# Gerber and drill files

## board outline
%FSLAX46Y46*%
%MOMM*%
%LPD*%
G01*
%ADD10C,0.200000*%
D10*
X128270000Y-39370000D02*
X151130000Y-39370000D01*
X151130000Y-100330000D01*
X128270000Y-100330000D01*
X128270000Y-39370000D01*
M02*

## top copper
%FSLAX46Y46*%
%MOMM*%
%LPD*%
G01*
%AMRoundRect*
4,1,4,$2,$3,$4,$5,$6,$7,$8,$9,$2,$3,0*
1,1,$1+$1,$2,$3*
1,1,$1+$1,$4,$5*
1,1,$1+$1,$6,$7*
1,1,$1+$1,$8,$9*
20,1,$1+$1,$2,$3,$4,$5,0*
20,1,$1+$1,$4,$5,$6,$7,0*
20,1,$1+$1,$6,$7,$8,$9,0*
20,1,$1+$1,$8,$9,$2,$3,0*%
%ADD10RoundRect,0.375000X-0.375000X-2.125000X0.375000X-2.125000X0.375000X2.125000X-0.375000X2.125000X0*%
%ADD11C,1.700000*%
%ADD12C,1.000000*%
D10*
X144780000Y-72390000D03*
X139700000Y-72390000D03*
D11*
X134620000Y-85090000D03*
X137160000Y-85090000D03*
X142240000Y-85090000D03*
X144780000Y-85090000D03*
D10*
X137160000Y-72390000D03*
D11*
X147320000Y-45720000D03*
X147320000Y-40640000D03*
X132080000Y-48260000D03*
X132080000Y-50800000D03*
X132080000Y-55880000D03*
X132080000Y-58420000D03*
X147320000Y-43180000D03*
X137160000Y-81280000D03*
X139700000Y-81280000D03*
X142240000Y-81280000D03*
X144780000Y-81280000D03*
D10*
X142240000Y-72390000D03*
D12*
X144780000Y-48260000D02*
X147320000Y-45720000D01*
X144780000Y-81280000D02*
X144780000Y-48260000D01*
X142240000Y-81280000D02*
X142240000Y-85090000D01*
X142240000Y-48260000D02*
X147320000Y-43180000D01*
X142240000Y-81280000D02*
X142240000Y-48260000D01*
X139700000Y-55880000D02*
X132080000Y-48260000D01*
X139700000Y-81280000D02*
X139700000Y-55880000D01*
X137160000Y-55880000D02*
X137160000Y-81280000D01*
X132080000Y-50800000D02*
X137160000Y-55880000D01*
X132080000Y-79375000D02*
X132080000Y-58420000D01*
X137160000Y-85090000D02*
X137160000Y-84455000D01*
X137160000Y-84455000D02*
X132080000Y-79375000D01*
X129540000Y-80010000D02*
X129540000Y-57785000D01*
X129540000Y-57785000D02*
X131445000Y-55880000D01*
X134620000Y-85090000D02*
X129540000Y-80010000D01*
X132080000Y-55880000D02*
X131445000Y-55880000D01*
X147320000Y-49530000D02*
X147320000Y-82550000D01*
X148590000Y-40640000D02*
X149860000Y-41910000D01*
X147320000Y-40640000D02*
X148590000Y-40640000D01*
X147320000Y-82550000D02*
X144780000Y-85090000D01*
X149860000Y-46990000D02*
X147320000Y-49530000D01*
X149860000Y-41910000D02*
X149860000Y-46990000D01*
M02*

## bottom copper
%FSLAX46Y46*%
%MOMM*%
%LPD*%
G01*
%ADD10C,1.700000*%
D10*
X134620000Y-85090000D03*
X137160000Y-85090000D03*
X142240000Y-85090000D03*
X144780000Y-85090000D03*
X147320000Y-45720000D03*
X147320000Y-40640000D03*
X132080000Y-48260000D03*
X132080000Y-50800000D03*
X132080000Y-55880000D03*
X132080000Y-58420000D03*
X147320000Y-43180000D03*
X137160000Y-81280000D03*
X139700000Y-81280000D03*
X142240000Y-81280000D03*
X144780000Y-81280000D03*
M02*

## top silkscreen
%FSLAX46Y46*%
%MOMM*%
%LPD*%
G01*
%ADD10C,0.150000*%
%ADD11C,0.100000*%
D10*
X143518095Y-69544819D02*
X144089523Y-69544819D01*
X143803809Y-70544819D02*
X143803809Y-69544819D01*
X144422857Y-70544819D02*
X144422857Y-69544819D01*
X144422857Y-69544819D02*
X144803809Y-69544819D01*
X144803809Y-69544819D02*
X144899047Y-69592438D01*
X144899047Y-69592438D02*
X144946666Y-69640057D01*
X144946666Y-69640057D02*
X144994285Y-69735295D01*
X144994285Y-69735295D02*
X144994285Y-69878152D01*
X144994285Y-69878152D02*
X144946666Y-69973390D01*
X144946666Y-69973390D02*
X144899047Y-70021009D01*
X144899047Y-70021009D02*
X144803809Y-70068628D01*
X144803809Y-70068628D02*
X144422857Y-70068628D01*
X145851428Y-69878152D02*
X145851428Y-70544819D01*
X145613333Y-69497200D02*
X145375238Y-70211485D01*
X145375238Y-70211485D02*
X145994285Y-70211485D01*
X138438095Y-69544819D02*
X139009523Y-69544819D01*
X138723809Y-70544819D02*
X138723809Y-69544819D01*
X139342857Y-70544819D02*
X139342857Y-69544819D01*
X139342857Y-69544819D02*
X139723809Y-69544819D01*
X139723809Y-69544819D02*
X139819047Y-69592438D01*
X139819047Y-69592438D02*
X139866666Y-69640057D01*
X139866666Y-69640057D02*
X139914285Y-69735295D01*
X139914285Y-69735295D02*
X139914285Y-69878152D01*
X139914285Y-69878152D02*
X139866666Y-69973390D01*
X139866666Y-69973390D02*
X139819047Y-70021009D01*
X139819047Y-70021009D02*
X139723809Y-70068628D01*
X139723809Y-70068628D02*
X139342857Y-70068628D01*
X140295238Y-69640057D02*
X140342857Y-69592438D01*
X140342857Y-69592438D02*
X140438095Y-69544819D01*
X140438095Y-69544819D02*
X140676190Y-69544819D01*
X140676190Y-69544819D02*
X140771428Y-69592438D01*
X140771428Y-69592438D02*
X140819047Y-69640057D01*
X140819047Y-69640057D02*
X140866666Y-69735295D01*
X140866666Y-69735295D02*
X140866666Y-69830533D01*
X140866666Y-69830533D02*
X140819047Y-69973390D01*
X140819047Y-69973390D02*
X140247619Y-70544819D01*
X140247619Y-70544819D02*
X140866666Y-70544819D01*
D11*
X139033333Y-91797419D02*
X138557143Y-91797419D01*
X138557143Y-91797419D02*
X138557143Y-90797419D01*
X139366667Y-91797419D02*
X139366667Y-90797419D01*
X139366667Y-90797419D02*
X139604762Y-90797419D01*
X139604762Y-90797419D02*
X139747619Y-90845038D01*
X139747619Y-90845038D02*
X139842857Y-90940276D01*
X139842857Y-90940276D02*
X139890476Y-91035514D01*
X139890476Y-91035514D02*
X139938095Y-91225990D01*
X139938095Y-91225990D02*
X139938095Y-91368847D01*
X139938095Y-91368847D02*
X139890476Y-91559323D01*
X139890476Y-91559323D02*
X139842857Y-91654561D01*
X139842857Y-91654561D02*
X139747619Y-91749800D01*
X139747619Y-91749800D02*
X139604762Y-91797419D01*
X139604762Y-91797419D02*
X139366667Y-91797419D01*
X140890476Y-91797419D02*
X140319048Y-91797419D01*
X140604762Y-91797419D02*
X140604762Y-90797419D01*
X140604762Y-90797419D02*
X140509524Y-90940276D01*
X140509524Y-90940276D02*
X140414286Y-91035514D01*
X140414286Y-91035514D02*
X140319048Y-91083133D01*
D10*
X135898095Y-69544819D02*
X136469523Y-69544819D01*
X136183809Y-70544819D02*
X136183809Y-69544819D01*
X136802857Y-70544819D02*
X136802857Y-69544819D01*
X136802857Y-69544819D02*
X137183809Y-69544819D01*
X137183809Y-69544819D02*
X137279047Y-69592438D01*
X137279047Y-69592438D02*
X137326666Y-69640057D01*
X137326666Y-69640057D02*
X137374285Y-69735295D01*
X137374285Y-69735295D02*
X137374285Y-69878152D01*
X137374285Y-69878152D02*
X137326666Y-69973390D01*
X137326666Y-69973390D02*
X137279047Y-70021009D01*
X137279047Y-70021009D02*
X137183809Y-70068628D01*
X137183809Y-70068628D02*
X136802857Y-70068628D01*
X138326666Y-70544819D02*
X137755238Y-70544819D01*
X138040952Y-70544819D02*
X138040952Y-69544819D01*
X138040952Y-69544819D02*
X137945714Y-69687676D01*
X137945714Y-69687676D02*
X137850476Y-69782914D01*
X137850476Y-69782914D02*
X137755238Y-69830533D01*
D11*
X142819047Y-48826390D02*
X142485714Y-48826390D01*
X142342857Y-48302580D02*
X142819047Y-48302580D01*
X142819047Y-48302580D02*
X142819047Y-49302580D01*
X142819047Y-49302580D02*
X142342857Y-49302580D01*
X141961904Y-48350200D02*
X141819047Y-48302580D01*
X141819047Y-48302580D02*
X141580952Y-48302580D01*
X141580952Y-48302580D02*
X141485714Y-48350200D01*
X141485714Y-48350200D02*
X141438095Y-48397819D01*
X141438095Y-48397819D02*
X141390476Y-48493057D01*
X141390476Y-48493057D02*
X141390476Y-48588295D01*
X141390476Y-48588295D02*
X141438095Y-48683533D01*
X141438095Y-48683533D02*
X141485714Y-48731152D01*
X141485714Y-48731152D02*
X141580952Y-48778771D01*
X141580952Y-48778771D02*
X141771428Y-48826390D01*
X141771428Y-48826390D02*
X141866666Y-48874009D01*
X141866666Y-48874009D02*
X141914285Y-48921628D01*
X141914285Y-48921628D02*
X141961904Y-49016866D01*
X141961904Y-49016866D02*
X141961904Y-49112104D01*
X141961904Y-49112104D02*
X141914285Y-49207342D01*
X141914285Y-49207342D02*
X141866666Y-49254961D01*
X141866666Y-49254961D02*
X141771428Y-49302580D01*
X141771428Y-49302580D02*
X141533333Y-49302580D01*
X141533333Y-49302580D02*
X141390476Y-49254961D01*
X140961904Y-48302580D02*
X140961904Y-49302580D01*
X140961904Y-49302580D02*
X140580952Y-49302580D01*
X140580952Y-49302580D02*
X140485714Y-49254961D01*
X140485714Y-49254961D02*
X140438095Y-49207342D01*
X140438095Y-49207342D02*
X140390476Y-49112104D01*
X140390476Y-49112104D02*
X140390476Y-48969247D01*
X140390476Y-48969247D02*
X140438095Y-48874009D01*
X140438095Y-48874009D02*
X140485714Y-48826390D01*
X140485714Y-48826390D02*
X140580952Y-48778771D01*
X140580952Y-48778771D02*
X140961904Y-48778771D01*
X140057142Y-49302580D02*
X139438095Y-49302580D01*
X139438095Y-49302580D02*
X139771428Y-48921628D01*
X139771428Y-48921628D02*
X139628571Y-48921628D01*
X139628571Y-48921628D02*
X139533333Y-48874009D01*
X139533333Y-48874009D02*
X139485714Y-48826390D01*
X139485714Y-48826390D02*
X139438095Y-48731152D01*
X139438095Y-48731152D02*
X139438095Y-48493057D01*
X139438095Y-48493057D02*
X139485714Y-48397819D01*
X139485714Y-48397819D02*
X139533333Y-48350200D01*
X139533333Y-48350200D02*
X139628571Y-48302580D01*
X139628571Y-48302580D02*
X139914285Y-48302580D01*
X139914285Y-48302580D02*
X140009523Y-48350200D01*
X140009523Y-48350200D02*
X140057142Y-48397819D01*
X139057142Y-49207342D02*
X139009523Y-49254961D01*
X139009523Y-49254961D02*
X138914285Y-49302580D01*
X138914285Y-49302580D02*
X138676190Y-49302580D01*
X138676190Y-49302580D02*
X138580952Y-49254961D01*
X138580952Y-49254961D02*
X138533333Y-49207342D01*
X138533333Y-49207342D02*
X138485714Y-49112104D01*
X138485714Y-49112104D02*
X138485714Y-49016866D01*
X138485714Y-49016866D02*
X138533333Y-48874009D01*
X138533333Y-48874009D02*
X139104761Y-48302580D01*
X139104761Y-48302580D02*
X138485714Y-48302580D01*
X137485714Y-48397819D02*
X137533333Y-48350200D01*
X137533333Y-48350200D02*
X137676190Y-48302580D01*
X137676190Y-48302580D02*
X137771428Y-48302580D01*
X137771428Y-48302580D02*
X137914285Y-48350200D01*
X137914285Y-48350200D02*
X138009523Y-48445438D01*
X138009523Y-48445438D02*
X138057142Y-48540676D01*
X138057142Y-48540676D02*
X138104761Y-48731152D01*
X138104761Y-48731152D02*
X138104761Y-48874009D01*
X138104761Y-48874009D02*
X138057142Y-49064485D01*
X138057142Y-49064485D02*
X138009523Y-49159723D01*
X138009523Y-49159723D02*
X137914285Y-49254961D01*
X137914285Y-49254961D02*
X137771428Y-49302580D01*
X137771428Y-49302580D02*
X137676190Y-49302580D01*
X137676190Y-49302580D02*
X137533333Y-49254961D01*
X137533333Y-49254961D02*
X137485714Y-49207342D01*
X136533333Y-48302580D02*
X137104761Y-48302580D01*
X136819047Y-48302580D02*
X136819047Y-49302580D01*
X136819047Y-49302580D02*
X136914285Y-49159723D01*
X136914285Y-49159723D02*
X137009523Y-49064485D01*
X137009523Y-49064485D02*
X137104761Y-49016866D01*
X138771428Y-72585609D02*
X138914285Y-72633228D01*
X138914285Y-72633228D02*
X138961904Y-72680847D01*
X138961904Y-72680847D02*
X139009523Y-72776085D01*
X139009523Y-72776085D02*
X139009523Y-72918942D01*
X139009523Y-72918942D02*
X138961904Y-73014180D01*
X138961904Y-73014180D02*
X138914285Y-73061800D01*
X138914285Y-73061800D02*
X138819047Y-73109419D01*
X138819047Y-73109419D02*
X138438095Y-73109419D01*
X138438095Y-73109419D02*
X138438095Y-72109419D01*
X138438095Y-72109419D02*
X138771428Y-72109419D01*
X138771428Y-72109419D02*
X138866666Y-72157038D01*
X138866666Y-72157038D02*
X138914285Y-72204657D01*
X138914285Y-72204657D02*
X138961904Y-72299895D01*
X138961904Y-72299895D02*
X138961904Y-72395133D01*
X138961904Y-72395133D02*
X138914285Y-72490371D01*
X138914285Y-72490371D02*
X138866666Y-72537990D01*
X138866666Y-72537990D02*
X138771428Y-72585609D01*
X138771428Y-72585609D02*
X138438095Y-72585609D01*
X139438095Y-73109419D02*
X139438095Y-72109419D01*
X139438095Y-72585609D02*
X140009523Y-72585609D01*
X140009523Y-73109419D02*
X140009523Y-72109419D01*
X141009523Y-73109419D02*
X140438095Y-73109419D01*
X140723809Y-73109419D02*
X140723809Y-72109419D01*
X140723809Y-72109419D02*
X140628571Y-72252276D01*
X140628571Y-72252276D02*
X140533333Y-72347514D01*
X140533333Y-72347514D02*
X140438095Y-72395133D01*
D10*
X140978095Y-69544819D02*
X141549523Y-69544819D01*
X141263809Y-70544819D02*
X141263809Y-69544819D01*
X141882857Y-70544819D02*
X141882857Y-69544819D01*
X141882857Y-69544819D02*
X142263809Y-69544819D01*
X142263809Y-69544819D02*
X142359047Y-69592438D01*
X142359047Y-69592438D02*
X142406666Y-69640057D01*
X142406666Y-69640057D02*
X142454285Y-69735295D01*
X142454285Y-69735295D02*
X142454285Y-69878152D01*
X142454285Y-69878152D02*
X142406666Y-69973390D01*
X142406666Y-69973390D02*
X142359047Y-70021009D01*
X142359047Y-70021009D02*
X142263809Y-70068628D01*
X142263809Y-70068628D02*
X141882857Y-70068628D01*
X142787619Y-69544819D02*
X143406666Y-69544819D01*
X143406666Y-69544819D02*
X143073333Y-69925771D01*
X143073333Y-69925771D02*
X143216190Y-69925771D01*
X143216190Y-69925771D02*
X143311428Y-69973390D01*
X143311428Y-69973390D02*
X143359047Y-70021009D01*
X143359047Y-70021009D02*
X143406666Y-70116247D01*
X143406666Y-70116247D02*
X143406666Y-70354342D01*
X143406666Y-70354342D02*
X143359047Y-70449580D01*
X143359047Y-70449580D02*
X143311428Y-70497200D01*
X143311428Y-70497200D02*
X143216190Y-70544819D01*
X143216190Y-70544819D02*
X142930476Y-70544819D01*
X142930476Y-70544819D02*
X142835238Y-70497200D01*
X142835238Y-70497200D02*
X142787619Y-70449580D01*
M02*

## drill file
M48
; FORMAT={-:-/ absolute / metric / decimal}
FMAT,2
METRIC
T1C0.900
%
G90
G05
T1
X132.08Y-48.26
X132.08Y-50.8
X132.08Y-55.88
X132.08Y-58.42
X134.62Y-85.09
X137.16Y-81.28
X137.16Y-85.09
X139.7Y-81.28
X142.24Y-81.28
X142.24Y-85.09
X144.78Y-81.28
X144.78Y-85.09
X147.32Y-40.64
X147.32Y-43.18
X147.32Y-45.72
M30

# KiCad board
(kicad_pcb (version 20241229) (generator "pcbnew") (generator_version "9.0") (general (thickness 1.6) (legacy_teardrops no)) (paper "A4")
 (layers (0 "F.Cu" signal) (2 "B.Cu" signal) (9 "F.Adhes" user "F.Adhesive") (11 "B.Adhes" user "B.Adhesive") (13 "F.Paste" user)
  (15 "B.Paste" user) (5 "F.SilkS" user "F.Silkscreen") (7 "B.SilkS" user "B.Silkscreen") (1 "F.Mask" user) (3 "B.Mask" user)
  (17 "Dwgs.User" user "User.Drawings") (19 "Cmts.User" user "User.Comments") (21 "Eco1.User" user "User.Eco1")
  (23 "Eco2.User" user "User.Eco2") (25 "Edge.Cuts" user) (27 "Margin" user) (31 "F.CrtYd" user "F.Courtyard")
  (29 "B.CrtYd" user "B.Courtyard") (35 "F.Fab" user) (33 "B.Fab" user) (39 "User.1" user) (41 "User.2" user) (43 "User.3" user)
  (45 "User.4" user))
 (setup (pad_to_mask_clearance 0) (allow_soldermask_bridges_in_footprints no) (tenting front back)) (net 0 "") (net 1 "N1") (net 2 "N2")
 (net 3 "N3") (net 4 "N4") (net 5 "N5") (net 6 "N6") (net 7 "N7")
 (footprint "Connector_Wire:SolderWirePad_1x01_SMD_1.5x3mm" (layer "F.Cu") (at 144.78 72.39)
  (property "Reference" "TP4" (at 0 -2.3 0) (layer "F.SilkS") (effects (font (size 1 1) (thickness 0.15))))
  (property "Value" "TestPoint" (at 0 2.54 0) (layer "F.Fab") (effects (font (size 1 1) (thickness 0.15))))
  (pad "1" smd roundrect (at 0 0) (size 1.5 5) (layers "F.Cu" "F.Mask") (roundrect_rratio 0.25) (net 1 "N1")))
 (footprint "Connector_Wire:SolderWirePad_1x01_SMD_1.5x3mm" (layer "F.Cu") (at 139.7 72.39)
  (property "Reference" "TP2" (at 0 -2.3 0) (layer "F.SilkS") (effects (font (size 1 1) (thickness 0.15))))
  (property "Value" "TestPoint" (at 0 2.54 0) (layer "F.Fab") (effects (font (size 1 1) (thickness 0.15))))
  (pad "1" smd roundrect (at 0 0) (size 1.5 5) (layers "F.Cu" "F.Mask") (roundrect_rratio 0.25) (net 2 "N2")))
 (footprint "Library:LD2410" (layer "F.Cu") (at 139.7 91.84)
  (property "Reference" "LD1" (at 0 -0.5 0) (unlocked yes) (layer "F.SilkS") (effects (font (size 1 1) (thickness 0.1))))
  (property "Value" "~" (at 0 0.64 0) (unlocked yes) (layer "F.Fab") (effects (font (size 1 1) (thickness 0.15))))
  (pad "1" thru_hole circle (at -5.08 -6.75 90) (size 1.7 1.7) (drill 0.9) (layers "*.Cu" "*.Mask") (remove_unused_layers yes)
   (keep_end_layers yes) (zone_layer_connections) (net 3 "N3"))
  (pad "2" thru_hole circle (at -2.54 -6.75 90) (size 1.7 1.7) (drill 0.9) (layers "*.Cu" "*.Mask") (remove_unused_layers yes)
   (keep_end_layers yes) (zone_layer_connections) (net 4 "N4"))
  (pad "4" thru_hole circle (at 2.54 -6.75 90) (size 1.7 1.7) (drill 0.9) (layers "*.Cu" "*.Mask") (remove_unused_layers yes)
   (keep_end_layers yes) (zone_layer_connections) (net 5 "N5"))
  (pad "5" thru_hole circle (at 5.08 -6.75 90) (size 1.7 1.7) (drill 0.9) (layers "*.Cu" "*.Mask") (remove_unused_layers yes)
   (keep_end_layers yes) (zone_layer_connections) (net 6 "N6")))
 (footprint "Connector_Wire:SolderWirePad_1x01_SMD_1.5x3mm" (layer "F.Cu") (at 137.16 72.39)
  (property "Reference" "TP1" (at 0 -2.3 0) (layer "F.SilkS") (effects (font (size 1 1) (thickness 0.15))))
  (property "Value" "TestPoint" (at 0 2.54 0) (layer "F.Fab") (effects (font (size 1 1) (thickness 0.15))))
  (pad "1" smd roundrect (at 0 0) (size 1.5 5) (layers "F.Cu" "F.Mask") (roundrect_rratio 0.25) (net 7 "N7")))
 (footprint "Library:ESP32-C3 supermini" (layer "F.Cu") (at 139.7 50.8 180)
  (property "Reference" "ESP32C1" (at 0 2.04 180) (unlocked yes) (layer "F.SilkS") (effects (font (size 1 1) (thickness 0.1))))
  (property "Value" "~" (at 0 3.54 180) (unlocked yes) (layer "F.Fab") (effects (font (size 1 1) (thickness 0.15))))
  (pad "3.3V" thru_hole circle (at -7.62 5.08 180) (size 1.7 1.7) (drill 0.9) (layers "*.Cu" "*.Mask") (remove_unused_layers yes)
   (keep_end_layers yes) (zone_layer_connections) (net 1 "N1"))
  (pad "5V" thru_hole circle (at -7.62 10.16 180) (size 1.7 1.7) (drill 0.9) (layers "*.Cu" "*.Mask") (remove_unused_layers yes)
   (keep_end_layers yes) (zone_layer_connections) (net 6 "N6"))
  (pad "8" thru_hole circle (at 7.62 2.54 180) (size 1.7 1.7) (drill 0.9) (layers "*.Cu" "*.Mask") (remove_unused_layers yes)
   (keep_end_layers yes) (zone_layer_connections) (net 2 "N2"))
  (pad "9" thru_hole circle (at 7.62 0 180) (size 1.7 1.7) (drill 0.9) (layers "*.Cu" "*.Mask") (remove_unused_layers yes)
   (keep_end_layers yes) (zone_layer_connections) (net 7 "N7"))
  (pad "20" thru_hole circle (at 7.62 -5.08 180) (size 1.7 1.7) (drill 0.9) (layers "*.Cu" "*.Mask") (remove_unused_layers yes)
   (keep_end_layers yes) (zone_layer_connections) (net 3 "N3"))
  (pad "21" thru_hole circle (at 7.62 -7.62 180) (size 1.7 1.7) (drill 0.9) (layers "*.Cu" "*.Mask") (remove_unused_layers yes)
   (keep_end_layers yes) (zone_layer_connections) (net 4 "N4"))
  (pad "GND" thru_hole circle (at -7.62 7.62 180) (size 1.7 1.7) (drill 0.9) (layers "*.Cu" "*.Mask") (remove_unused_layers yes)
   (keep_end_layers yes) (zone_layer_connections) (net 5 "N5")))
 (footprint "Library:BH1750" (layer "F.Cu") (at 139.7 73.152)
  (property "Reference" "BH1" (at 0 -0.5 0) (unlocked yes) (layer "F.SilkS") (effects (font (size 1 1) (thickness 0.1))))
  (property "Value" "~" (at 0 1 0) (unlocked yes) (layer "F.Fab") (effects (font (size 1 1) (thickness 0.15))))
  (pad "1" thru_hole circle (at -2.54 8.128 90) (size 1.7 1.7) (drill 0.9) (layers "*.Cu" "*.Mask") (remove_unused_layers yes)
   (keep_end_layers yes) (zone_layer_connections) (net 7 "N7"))
  (pad "2" thru_hole circle (at 0 8.128 90) (size 1.7 1.7) (drill 0.9) (layers "*.Cu" "*.Mask") (remove_unused_layers yes)
   (keep_end_layers yes) (zone_layer_connections) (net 2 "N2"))
  (pad "3" thru_hole circle (at 2.54 8.128 90) (size 1.7 1.7) (drill 0.9) (layers "*.Cu" "*.Mask") (remove_unused_layers yes)
   (keep_end_layers yes) (zone_layer_connections) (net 5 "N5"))
  (pad "4" thru_hole circle (at 5.08 8.128 90) (size 1.7 1.7) (drill 0.9) (layers "*.Cu" "*.Mask") (remove_unused_layers yes)
   (keep_end_layers yes) (zone_layer_connections) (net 1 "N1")))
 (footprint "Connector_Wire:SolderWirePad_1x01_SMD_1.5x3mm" (layer "F.Cu") (at 142.24 72.39)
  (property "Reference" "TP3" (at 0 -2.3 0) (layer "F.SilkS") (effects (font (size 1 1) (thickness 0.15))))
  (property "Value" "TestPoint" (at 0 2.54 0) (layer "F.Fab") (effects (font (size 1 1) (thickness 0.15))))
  (pad "1" smd roundrect (at 0 0) (size 1.5 5) (layers "F.Cu" "F.Mask") (roundrect_rratio 0.25) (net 5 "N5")))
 (gr_rect (start 128.27 39.37) (end 151.13 100.33) (stroke (width 0.2) (type solid)) (fill no) (layer "Edge.Cuts"))
 (segment (start 144.78 48.26) (end 147.32 45.72) (width 1) (layer "F.Cu") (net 1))
 (segment (start 144.78 81.28) (end 144.78 48.26) (width 1) (layer "F.Cu") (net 1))
 (segment (start 142.24 81.28) (end 142.24 85.09) (width 1) (layer "F.Cu") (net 5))
 (segment (start 142.24 48.26) (end 147.32 43.18) (width 1) (layer "F.Cu") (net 5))
 (segment (start 142.24 81.28) (end 142.24 48.26) (width 1) (layer "F.Cu") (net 5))
 (segment (start 139.7 55.88) (end 132.08 48.26) (width 1) (layer "F.Cu") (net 2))
 (segment (start 139.7 81.28) (end 139.7 55.88) (width 1) (layer "F.Cu") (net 2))
 (segment (start 137.16 55.88) (end 137.16 81.28) (width 1) (layer "F.Cu") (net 7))
 (segment (start 132.08 50.8) (end 137.16 55.88) (width 1) (layer "F.Cu") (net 7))
 (segment (start 132.08 79.375) (end 132.08 58.42) (width 1) (layer "F.Cu") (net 4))
 (segment (start 137.16 85.09) (end 137.16 84.455) (width 1) (layer "F.Cu") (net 4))
 (segment (start 137.16 84.455) (end 132.08 79.375) (width 1) (layer "F.Cu") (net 4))
 (segment (start 129.54 80.01) (end 129.54 57.785) (width 1) (layer "F.Cu") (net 3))
 (segment (start 129.54 57.785) (end 131.445 55.88) (width 1) (layer "F.Cu") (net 3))
 (segment (start 134.62 85.09) (end 129.54 80.01) (width 1) (layer "F.Cu") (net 3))
 (segment (start 132.08 55.88) (end 131.445 55.88) (width 1) (layer "F.Cu") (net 3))
 (segment (start 147.32 49.53) (end 147.32 82.55) (width 1) (layer "F.Cu") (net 6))
 (segment (start 148.59 40.64) (end 149.86 41.91) (width 1) (layer "F.Cu") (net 6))
 (segment (start 147.32 40.64) (end 148.59 40.64) (width 1) (layer "F.Cu") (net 6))
 (segment (start 147.32 82.55) (end 144.78 85.09) (width 1) (layer "F.Cu") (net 6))
 (segment (start 149.86 46.99) (end 147.32 49.53) (width 1) (layer "F.Cu") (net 6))
 (segment (start 149.86 41.91) (end 149.86 46.99) (width 1) (layer "F.Cu") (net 6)))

